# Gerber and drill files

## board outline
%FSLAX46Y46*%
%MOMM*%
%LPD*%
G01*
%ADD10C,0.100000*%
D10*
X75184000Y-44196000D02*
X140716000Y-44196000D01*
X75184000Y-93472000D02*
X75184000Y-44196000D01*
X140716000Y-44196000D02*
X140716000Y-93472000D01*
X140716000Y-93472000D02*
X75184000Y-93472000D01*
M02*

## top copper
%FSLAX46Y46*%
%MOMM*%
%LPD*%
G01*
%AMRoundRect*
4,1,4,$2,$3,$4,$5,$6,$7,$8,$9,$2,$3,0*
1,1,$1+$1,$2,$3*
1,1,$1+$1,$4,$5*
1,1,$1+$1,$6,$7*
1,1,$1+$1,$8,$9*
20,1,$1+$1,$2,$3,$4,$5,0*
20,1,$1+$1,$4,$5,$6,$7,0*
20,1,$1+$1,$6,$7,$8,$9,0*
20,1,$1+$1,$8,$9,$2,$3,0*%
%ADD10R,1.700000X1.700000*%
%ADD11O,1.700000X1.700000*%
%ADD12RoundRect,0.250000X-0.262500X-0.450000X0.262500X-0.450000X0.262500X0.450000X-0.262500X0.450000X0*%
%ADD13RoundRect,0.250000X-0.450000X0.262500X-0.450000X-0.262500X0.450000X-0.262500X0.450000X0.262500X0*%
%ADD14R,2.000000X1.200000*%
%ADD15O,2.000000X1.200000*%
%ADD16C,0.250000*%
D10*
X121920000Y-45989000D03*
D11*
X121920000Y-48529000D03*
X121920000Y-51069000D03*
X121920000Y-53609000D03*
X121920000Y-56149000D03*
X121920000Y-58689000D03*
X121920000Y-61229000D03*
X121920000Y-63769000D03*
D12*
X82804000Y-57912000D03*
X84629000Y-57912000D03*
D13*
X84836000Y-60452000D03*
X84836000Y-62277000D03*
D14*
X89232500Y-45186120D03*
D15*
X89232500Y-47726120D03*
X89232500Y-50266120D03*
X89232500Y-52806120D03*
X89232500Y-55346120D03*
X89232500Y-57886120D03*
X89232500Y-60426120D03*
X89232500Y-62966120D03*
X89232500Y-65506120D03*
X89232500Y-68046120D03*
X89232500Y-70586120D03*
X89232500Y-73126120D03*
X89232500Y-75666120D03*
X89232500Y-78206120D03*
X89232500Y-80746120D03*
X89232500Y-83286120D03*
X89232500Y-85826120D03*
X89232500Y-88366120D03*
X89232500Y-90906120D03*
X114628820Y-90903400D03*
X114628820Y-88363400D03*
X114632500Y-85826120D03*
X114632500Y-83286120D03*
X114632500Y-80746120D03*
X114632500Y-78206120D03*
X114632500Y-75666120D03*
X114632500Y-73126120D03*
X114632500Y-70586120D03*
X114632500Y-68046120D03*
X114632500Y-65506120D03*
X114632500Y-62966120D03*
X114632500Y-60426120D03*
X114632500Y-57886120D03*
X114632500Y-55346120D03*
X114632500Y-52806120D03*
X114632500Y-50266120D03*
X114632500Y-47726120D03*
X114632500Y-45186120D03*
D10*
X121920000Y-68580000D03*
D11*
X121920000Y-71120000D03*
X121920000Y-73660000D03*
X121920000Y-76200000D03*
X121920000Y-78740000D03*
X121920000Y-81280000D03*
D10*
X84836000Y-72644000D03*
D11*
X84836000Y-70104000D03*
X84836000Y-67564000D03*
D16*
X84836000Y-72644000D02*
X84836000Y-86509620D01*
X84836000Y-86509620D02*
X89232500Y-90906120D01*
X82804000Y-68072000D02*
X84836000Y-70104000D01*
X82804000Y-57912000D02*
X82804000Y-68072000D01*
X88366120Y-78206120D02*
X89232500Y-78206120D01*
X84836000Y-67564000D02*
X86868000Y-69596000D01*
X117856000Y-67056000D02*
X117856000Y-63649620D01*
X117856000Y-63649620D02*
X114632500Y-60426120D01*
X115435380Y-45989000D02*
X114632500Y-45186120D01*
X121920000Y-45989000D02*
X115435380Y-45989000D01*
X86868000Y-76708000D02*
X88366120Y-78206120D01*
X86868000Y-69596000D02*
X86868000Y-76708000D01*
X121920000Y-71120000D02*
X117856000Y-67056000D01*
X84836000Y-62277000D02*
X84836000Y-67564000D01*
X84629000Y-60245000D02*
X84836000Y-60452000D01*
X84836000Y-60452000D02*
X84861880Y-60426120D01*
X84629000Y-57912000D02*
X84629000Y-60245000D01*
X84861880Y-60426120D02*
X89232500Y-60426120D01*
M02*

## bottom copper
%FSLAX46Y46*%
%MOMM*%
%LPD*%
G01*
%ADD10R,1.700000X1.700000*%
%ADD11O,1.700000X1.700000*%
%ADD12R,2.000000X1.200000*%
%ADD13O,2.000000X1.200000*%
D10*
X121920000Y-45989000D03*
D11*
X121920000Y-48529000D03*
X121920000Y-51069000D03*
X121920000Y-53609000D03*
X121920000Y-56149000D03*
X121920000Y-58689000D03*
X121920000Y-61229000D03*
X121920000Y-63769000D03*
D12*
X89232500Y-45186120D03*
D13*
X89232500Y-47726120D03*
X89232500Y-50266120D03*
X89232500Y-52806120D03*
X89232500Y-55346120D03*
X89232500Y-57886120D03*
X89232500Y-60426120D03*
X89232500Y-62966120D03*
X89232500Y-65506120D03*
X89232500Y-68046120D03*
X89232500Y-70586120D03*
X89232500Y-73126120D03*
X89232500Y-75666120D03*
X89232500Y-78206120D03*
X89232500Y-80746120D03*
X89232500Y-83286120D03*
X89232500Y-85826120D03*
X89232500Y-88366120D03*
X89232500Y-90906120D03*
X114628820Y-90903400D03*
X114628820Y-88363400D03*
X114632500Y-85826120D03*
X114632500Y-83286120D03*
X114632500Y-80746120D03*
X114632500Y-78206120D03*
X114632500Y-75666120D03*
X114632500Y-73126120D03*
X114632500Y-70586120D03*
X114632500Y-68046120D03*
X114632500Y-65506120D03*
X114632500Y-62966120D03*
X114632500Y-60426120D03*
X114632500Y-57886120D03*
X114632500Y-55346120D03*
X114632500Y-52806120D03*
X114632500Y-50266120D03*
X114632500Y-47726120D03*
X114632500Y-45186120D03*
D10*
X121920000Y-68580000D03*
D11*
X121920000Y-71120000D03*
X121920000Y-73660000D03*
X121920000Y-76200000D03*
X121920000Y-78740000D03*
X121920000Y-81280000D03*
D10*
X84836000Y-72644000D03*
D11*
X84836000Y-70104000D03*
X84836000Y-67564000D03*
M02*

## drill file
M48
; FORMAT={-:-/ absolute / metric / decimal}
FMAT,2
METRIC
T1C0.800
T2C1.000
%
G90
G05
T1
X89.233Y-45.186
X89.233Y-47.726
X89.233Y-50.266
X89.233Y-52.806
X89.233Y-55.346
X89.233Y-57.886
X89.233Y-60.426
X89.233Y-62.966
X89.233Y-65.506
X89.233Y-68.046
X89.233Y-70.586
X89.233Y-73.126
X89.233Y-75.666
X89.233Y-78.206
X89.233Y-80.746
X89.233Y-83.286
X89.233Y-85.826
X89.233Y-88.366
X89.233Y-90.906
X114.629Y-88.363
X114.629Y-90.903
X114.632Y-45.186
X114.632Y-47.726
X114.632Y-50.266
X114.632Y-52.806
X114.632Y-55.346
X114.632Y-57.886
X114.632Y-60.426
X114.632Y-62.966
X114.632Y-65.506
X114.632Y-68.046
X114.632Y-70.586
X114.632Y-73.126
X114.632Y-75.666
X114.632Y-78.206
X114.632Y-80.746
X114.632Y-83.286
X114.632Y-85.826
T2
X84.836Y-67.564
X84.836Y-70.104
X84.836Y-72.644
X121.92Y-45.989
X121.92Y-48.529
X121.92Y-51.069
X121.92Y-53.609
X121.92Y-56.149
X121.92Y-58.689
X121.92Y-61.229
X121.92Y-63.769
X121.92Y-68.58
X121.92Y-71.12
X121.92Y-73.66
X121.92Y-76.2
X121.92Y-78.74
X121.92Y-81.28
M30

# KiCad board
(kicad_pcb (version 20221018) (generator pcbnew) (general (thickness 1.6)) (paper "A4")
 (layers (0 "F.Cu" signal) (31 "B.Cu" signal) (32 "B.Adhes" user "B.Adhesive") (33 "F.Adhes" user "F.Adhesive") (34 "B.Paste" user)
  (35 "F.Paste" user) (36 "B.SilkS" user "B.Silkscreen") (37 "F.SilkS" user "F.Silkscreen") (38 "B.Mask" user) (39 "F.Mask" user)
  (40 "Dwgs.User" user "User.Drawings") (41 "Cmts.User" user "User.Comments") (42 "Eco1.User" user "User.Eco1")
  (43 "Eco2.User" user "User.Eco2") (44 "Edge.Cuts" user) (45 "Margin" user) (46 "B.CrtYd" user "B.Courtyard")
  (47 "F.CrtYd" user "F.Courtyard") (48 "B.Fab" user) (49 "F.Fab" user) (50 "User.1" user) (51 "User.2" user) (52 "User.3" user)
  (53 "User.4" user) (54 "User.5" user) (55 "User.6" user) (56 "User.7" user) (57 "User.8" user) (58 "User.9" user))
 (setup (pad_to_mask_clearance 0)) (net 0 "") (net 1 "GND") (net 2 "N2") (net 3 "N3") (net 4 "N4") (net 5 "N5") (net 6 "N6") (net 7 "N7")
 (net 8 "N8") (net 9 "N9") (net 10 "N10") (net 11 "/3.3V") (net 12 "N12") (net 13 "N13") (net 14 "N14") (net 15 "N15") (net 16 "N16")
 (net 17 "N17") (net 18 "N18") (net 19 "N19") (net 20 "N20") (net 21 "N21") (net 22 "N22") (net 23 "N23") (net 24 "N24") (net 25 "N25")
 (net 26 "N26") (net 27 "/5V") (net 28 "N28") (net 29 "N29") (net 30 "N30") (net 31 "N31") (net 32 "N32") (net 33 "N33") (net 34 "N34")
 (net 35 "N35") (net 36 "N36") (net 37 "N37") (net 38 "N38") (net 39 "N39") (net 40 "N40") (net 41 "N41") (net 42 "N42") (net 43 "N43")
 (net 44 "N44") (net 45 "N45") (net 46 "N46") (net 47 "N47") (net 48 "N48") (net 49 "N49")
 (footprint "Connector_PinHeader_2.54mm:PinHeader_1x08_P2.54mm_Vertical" (layer "F.Cu") (at 121.92 45.989)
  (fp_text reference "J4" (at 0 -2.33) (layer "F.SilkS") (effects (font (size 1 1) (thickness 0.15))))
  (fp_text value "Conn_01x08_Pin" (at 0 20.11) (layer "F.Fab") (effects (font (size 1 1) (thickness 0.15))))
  (pad "1" thru_hole rect (at 0 0) (size 1.7 1.7) (drill 1) (layers "*.Cu" "*.Mask") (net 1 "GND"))
  (pad "2" thru_hole oval (at 0 2.54) (size 1.7 1.7) (drill 1) (layers "*.Cu" "*.Mask") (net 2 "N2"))
  (pad "3" thru_hole oval (at 0 5.08) (size 1.7 1.7) (drill 1) (layers "*.Cu" "*.Mask") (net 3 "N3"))
  (pad "4" thru_hole oval (at 0 7.62) (size 1.7 1.7) (drill 1) (layers "*.Cu" "*.Mask") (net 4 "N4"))
  (pad "5" thru_hole oval (at 0 10.16) (size 1.7 1.7) (drill 1) (layers "*.Cu" "*.Mask") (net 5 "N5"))
  (pad "6" thru_hole oval (at 0 12.7) (size 1.7 1.7) (drill 1) (layers "*.Cu" "*.Mask") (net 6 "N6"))
  (pad "7" thru_hole oval (at 0 15.24) (size 1.7 1.7) (drill 1) (layers "*.Cu" "*.Mask") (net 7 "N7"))
  (pad "8" thru_hole oval (at 0 17.78) (size 1.7 1.7) (drill 1) (layers "*.Cu" "*.Mask") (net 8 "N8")))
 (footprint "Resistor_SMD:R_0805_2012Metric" (layer "F.Cu") (at 83.7165 57.912)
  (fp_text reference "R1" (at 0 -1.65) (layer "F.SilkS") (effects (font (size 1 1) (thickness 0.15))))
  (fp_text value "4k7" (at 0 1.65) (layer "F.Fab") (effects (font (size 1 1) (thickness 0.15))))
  (pad "1" smd roundrect (at -0.9125 0) (size 1.025 1.4) (layers "F.Cu" "F.Paste" "F.Mask") (roundrect_rratio 0.243902) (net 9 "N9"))
  (pad "2" smd roundrect (at 0.9125 0) (size 1.025 1.4) (layers "F.Cu" "F.Paste" "F.Mask") (roundrect_rratio 0.243902) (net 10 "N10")))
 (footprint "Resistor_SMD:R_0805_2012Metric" (layer "F.Cu") (at 84.836 61.3645 -90)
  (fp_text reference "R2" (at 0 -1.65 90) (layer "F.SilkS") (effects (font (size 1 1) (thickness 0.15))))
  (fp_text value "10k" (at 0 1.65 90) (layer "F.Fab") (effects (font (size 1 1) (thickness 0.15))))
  (pad "1" smd roundrect (at -0.9125 0 270) (size 1.025 1.4) (layers "F.Cu" "F.Paste" "F.Mask") (roundrect_rratio 0.243902) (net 10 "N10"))
  (pad "2" smd roundrect (at 0.9125 0 270) (size 1.025 1.4) (layers "F.Cu" "F.Paste" "F.Mask") (roundrect_rratio 0.243902) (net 1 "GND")))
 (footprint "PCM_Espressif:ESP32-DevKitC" (layer "F.Cu") (at 89.2325 45.18612)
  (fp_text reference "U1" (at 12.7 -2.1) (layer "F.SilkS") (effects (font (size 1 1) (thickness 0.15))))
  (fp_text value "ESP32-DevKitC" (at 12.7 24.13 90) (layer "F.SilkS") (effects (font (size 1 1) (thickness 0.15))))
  (pad "1" thru_hole rect (at 0 0 270) (size 1.2 2) (drill 0.8) (layers "*.Cu" "*.Mask") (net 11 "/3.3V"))
  (pad "2" thru_hole oval (at 0 2.54 270) (size 1.2 2) (drill 0.8) (layers "*.Cu" "*.Mask") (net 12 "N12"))
  (pad "3" thru_hole oval (at 0 5.08 270) (size 1.2 2) (drill 0.8) (layers "*.Cu" "*.Mask") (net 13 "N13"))
  (pad "4" thru_hole oval (at 0 7.62 270) (size 1.2 2) (drill 0.8) (layers "*.Cu" "*.Mask") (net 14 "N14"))
  (pad "5" thru_hole oval (at 0 10.16 270) (size 1.2 2) (drill 0.8) (layers "*.Cu" "*.Mask") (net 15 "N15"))
  (pad "6" thru_hole oval (at 0 12.7 270) (size 1.2 2) (drill 0.8) (layers "*.Cu" "*.Mask") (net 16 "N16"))
  (pad "7" thru_hole oval (at 0 15.24 270) (size 1.2 2) (drill 0.8) (layers "*.Cu" "*.Mask") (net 10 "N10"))
  (pad "8" thru_hole oval (at 0 17.78 270) (size 1.2 2) (drill 0.8) (layers "*.Cu" "*.Mask") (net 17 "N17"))
  (pad "9" thru_hole oval (at 0 20.32 270) (size 1.2 2) (drill 0.8) (layers "*.Cu" "*.Mask") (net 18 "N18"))
  (pad "10" thru_hole oval (at 0 22.86 270) (size 1.2 2) (drill 0.8) (layers "*.Cu" "*.Mask") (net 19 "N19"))
  (pad "11" thru_hole oval (at 0 25.4 270) (size 1.2 2) (drill 0.8) (layers "*.Cu" "*.Mask") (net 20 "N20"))
  (pad "12" thru_hole oval (at 0 27.94 270) (size 1.2 2) (drill 0.8) (layers "*.Cu" "*.Mask") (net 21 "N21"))
  (pad "13" thru_hole oval (at 0 30.48 270) (size 1.2 2) (drill 0.8) (layers "*.Cu" "*.Mask") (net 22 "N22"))
  (pad "14" thru_hole oval (at 0 33.02 270) (size 1.2 2) (drill 0.8) (layers "*.Cu" "*.Mask") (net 1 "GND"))
  (pad "15" thru_hole oval (at 0 35.56 270) (size 1.2 2) (drill 0.8) (layers "*.Cu" "*.Mask") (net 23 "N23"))
  (pad "16" thru_hole oval (at 0 38.1 270) (size 1.2 2) (drill 0.8) (layers "*.Cu" "*.Mask") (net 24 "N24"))
  (pad "17" thru_hole oval (at 0 40.64 270) (size 1.2 2) (drill 0.8) (layers "*.Cu" "*.Mask") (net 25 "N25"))
  (pad "18" thru_hole oval (at 0 43.18 270) (size 1.2 2) (drill 0.8) (layers "*.Cu" "*.Mask") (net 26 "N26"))
  (pad "19" thru_hole oval (at 0 45.72 270) (size 1.2 2) (drill 0.8) (layers "*.Cu" "*.Mask") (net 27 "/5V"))
  (pad "20" thru_hole oval (at 25.39632 45.71728 270) (size 1.2 2) (drill 0.8) (layers "*.Cu" "*.Mask") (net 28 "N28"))
  (pad "21" thru_hole oval (at 25.39632 43.17728 270) (size 1.2 2) (drill 0.8) (layers "*.Cu" "*.Mask") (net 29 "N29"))
  (pad "22" thru_hole oval (at 25.4 40.64 270) (size 1.2 2) (drill 0.8) (layers "*.Cu" "*.Mask") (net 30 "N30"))
  (pad "23" thru_hole oval (at 25.4 38.1 270) (size 1.2 2) (drill 0.8) (layers "*.Cu" "*.Mask") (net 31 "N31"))
  (pad "24" thru_hole oval (at 25.4 35.56 270) (size 1.2 2) (drill 0.8) (layers "*.Cu" "*.Mask") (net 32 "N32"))
  (pad "25" thru_hole oval (at 25.4 33.02 270) (size 1.2 2) (drill 0.8) (layers "*.Cu" "*.Mask") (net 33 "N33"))
  (pad "26" thru_hole oval (at 25.4 30.48 270) (size 1.2 2) (drill 0.8) (layers "*.Cu" "*.Mask") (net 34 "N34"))
  (pad "27" thru_hole oval (at 25.4 27.94 270) (size 1.2 2) (drill 0.8) (layers "*.Cu" "*.Mask") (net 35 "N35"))
  (pad "28" thru_hole oval (at 25.4 25.4 270) (size 1.2 2) (drill 0.8) (layers "*.Cu" "*.Mask") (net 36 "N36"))
  (pad "29" thru_hole oval (at 25.4 22.86 270) (size 1.2 2) (drill 0.8) (layers "*.Cu" "*.Mask") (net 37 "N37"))
  (pad "30" thru_hole oval (at 25.4 20.32 270) (size 1.2 2) (drill 0.8) (layers "*.Cu" "*.Mask") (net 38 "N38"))
  (pad "31" thru_hole oval (at 25.4 17.78 270) (size 1.2 2) (drill 0.8) (layers "*.Cu" "*.Mask") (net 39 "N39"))
  (pad "32" thru_hole oval (at 25.4 15.24 270) (size 1.2 2) (drill 0.8) (layers "*.Cu" "*.Mask") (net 1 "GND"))
  (pad "33" thru_hole oval (at 25.4 12.7 270) (size 1.2 2) (drill 0.8) (layers "*.Cu" "*.Mask") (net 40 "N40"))
  (pad "34" thru_hole oval (at 25.4 10.16 270) (size 1.2 2) (drill 0.8) (layers "*.Cu" "*.Mask") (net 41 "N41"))
  (pad "35" thru_hole oval (at 25.4 7.62 270) (size 1.2 2) (drill 0.8) (layers "*.Cu" "*.Mask") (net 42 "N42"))
  (pad "36" thru_hole oval (at 25.4 5.08 270) (size 1.2 2) (drill 0.8) (layers "*.Cu" "*.Mask") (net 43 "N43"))
  (pad "37" thru_hole oval (at 25.4 2.54 270) (size 1.2 2) (drill 0.8) (layers "*.Cu" "*.Mask") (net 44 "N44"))
  (pad "38" thru_hole oval (at 25.4 0 270) (size 1.2 2) (drill 0.8) (layers "*.Cu" "*.Mask") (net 1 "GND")))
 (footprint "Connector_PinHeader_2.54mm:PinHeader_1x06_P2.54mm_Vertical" (layer "F.Cu") (at 121.92 68.58)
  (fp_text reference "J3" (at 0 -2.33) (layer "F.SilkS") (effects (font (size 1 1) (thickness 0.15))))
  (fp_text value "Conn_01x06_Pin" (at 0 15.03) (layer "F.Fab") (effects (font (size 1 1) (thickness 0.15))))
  (pad "1" thru_hole rect (at 0 0) (size 1.7 1.7) (drill 1) (layers "*.Cu" "*.Mask") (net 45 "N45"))
  (pad "2" thru_hole oval (at 0 2.54) (size 1.7 1.7) (drill 1) (layers "*.Cu" "*.Mask") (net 1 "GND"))
  (pad "3" thru_hole oval (at 0 5.08) (size 1.7 1.7) (drill 1) (layers "*.Cu" "*.Mask") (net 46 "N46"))
  (pad "4" thru_hole oval (at 0 7.62) (size 1.7 1.7) (drill 1) (layers "*.Cu" "*.Mask") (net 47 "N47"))
  (pad "5" thru_hole oval (at 0 10.16) (size 1.7 1.7) (drill 1) (layers "*.Cu" "*.Mask") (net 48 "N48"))
  (pad "6" thru_hole oval (at 0 12.7) (size 1.7 1.7) (drill 1) (layers "*.Cu" "*.Mask") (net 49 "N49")))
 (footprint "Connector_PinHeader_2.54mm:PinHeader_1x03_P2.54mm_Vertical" (layer "F.Cu") (at 84.836 72.644 180)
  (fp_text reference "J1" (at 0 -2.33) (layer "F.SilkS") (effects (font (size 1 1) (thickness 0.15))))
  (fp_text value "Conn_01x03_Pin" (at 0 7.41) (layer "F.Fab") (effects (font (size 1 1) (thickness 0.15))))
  (pad "1" thru_hole rect (at 0 0 180) (size 1.7 1.7) (drill 1) (layers "*.Cu" "*.Mask") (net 27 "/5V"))
  (pad "2" thru_hole oval (at 0 2.54 180) (size 1.7 1.7) (drill 1) (layers "*.Cu" "*.Mask") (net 9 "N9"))
  (pad "3" thru_hole oval (at 0 5.08 180) (size 1.7 1.7) (drill 1) (layers "*.Cu" "*.Mask") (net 1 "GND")))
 (gr_line (start 75.184 44.196) (end 140.716 44.196) (stroke (width 0.1) (type default)) (layer "Edge.Cuts"))
 (gr_line (start 75.184 93.472) (end 75.184 44.196) (stroke (width 0.1) (type default)) (layer "Edge.Cuts"))
 (gr_line (start 140.716 44.196) (end 140.716 93.472) (stroke (width 0.1) (type default)) (layer "Edge.Cuts"))
 (gr_line (start 140.716 93.472) (end 75.184 93.472) (stroke (width 0.1) (type default)) (layer "Edge.Cuts"))
 (segment (start 84.836 72.644) (end 84.836 86.50962) (width 0.25) (layer "F.Cu") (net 27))
 (segment (start 84.836 86.50962) (end 89.2325 90.90612) (width 0.25) (layer "F.Cu") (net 27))
 (segment (start 82.804 68.072) (end 84.836 70.104) (width 0.25) (layer "F.Cu") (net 9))
 (segment (start 82.804 57.912) (end 82.804 68.072) (width 0.25) (layer "F.Cu") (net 9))
 (segment (start 88.36612 78.20612) (end 89.2325 78.20612) (width 0.25) (layer "F.Cu") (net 1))
 (segment (start 84.836 67.564) (end 86.868 69.596) (width 0.25) (layer "F.Cu") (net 1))
 (segment (start 117.856 67.056) (end 117.856 63.64962) (width 0.25) (layer "F.Cu") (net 1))
 (segment (start 117.856 63.64962) (end 114.6325 60.42612) (width 0.25) (layer "F.Cu") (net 1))
 (segment (start 115.43538 45.989) (end 114.6325 45.18612) (width 0.25) (layer "F.Cu") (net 1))
 (segment (start 121.92 45.989) (end 115.43538 45.989) (width 0.25) (layer "F.Cu") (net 1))
 (segment (start 86.868 76.708) (end 88.36612 78.20612) (width 0.25) (layer "F.Cu") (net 1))
 (segment (start 86.868 69.596) (end 86.868 76.708) (width 0.25) (layer "F.Cu") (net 1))
 (segment (start 121.92 71.12) (end 117.856 67.056) (width 0.25) (layer "F.Cu") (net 1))
 (segment (start 84.836 62.277) (end 84.836 67.564) (width 0.25) (layer "F.Cu") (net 1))
 (segment (start 84.629 60.245) (end 84.836 60.452) (width 0.25) (layer "F.Cu") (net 10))
 (segment (start 84.836 60.452) (end 84.86188 60.42612) (width 0.25) (layer "F.Cu") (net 10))
 (segment (start 84.629 57.912) (end 84.629 60.245) (width 0.25) (layer "F.Cu") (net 10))
 (segment (start 84.86188 60.42612) (end 89.2325 60.42612) (width 0.25) (layer "F.Cu") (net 10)))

